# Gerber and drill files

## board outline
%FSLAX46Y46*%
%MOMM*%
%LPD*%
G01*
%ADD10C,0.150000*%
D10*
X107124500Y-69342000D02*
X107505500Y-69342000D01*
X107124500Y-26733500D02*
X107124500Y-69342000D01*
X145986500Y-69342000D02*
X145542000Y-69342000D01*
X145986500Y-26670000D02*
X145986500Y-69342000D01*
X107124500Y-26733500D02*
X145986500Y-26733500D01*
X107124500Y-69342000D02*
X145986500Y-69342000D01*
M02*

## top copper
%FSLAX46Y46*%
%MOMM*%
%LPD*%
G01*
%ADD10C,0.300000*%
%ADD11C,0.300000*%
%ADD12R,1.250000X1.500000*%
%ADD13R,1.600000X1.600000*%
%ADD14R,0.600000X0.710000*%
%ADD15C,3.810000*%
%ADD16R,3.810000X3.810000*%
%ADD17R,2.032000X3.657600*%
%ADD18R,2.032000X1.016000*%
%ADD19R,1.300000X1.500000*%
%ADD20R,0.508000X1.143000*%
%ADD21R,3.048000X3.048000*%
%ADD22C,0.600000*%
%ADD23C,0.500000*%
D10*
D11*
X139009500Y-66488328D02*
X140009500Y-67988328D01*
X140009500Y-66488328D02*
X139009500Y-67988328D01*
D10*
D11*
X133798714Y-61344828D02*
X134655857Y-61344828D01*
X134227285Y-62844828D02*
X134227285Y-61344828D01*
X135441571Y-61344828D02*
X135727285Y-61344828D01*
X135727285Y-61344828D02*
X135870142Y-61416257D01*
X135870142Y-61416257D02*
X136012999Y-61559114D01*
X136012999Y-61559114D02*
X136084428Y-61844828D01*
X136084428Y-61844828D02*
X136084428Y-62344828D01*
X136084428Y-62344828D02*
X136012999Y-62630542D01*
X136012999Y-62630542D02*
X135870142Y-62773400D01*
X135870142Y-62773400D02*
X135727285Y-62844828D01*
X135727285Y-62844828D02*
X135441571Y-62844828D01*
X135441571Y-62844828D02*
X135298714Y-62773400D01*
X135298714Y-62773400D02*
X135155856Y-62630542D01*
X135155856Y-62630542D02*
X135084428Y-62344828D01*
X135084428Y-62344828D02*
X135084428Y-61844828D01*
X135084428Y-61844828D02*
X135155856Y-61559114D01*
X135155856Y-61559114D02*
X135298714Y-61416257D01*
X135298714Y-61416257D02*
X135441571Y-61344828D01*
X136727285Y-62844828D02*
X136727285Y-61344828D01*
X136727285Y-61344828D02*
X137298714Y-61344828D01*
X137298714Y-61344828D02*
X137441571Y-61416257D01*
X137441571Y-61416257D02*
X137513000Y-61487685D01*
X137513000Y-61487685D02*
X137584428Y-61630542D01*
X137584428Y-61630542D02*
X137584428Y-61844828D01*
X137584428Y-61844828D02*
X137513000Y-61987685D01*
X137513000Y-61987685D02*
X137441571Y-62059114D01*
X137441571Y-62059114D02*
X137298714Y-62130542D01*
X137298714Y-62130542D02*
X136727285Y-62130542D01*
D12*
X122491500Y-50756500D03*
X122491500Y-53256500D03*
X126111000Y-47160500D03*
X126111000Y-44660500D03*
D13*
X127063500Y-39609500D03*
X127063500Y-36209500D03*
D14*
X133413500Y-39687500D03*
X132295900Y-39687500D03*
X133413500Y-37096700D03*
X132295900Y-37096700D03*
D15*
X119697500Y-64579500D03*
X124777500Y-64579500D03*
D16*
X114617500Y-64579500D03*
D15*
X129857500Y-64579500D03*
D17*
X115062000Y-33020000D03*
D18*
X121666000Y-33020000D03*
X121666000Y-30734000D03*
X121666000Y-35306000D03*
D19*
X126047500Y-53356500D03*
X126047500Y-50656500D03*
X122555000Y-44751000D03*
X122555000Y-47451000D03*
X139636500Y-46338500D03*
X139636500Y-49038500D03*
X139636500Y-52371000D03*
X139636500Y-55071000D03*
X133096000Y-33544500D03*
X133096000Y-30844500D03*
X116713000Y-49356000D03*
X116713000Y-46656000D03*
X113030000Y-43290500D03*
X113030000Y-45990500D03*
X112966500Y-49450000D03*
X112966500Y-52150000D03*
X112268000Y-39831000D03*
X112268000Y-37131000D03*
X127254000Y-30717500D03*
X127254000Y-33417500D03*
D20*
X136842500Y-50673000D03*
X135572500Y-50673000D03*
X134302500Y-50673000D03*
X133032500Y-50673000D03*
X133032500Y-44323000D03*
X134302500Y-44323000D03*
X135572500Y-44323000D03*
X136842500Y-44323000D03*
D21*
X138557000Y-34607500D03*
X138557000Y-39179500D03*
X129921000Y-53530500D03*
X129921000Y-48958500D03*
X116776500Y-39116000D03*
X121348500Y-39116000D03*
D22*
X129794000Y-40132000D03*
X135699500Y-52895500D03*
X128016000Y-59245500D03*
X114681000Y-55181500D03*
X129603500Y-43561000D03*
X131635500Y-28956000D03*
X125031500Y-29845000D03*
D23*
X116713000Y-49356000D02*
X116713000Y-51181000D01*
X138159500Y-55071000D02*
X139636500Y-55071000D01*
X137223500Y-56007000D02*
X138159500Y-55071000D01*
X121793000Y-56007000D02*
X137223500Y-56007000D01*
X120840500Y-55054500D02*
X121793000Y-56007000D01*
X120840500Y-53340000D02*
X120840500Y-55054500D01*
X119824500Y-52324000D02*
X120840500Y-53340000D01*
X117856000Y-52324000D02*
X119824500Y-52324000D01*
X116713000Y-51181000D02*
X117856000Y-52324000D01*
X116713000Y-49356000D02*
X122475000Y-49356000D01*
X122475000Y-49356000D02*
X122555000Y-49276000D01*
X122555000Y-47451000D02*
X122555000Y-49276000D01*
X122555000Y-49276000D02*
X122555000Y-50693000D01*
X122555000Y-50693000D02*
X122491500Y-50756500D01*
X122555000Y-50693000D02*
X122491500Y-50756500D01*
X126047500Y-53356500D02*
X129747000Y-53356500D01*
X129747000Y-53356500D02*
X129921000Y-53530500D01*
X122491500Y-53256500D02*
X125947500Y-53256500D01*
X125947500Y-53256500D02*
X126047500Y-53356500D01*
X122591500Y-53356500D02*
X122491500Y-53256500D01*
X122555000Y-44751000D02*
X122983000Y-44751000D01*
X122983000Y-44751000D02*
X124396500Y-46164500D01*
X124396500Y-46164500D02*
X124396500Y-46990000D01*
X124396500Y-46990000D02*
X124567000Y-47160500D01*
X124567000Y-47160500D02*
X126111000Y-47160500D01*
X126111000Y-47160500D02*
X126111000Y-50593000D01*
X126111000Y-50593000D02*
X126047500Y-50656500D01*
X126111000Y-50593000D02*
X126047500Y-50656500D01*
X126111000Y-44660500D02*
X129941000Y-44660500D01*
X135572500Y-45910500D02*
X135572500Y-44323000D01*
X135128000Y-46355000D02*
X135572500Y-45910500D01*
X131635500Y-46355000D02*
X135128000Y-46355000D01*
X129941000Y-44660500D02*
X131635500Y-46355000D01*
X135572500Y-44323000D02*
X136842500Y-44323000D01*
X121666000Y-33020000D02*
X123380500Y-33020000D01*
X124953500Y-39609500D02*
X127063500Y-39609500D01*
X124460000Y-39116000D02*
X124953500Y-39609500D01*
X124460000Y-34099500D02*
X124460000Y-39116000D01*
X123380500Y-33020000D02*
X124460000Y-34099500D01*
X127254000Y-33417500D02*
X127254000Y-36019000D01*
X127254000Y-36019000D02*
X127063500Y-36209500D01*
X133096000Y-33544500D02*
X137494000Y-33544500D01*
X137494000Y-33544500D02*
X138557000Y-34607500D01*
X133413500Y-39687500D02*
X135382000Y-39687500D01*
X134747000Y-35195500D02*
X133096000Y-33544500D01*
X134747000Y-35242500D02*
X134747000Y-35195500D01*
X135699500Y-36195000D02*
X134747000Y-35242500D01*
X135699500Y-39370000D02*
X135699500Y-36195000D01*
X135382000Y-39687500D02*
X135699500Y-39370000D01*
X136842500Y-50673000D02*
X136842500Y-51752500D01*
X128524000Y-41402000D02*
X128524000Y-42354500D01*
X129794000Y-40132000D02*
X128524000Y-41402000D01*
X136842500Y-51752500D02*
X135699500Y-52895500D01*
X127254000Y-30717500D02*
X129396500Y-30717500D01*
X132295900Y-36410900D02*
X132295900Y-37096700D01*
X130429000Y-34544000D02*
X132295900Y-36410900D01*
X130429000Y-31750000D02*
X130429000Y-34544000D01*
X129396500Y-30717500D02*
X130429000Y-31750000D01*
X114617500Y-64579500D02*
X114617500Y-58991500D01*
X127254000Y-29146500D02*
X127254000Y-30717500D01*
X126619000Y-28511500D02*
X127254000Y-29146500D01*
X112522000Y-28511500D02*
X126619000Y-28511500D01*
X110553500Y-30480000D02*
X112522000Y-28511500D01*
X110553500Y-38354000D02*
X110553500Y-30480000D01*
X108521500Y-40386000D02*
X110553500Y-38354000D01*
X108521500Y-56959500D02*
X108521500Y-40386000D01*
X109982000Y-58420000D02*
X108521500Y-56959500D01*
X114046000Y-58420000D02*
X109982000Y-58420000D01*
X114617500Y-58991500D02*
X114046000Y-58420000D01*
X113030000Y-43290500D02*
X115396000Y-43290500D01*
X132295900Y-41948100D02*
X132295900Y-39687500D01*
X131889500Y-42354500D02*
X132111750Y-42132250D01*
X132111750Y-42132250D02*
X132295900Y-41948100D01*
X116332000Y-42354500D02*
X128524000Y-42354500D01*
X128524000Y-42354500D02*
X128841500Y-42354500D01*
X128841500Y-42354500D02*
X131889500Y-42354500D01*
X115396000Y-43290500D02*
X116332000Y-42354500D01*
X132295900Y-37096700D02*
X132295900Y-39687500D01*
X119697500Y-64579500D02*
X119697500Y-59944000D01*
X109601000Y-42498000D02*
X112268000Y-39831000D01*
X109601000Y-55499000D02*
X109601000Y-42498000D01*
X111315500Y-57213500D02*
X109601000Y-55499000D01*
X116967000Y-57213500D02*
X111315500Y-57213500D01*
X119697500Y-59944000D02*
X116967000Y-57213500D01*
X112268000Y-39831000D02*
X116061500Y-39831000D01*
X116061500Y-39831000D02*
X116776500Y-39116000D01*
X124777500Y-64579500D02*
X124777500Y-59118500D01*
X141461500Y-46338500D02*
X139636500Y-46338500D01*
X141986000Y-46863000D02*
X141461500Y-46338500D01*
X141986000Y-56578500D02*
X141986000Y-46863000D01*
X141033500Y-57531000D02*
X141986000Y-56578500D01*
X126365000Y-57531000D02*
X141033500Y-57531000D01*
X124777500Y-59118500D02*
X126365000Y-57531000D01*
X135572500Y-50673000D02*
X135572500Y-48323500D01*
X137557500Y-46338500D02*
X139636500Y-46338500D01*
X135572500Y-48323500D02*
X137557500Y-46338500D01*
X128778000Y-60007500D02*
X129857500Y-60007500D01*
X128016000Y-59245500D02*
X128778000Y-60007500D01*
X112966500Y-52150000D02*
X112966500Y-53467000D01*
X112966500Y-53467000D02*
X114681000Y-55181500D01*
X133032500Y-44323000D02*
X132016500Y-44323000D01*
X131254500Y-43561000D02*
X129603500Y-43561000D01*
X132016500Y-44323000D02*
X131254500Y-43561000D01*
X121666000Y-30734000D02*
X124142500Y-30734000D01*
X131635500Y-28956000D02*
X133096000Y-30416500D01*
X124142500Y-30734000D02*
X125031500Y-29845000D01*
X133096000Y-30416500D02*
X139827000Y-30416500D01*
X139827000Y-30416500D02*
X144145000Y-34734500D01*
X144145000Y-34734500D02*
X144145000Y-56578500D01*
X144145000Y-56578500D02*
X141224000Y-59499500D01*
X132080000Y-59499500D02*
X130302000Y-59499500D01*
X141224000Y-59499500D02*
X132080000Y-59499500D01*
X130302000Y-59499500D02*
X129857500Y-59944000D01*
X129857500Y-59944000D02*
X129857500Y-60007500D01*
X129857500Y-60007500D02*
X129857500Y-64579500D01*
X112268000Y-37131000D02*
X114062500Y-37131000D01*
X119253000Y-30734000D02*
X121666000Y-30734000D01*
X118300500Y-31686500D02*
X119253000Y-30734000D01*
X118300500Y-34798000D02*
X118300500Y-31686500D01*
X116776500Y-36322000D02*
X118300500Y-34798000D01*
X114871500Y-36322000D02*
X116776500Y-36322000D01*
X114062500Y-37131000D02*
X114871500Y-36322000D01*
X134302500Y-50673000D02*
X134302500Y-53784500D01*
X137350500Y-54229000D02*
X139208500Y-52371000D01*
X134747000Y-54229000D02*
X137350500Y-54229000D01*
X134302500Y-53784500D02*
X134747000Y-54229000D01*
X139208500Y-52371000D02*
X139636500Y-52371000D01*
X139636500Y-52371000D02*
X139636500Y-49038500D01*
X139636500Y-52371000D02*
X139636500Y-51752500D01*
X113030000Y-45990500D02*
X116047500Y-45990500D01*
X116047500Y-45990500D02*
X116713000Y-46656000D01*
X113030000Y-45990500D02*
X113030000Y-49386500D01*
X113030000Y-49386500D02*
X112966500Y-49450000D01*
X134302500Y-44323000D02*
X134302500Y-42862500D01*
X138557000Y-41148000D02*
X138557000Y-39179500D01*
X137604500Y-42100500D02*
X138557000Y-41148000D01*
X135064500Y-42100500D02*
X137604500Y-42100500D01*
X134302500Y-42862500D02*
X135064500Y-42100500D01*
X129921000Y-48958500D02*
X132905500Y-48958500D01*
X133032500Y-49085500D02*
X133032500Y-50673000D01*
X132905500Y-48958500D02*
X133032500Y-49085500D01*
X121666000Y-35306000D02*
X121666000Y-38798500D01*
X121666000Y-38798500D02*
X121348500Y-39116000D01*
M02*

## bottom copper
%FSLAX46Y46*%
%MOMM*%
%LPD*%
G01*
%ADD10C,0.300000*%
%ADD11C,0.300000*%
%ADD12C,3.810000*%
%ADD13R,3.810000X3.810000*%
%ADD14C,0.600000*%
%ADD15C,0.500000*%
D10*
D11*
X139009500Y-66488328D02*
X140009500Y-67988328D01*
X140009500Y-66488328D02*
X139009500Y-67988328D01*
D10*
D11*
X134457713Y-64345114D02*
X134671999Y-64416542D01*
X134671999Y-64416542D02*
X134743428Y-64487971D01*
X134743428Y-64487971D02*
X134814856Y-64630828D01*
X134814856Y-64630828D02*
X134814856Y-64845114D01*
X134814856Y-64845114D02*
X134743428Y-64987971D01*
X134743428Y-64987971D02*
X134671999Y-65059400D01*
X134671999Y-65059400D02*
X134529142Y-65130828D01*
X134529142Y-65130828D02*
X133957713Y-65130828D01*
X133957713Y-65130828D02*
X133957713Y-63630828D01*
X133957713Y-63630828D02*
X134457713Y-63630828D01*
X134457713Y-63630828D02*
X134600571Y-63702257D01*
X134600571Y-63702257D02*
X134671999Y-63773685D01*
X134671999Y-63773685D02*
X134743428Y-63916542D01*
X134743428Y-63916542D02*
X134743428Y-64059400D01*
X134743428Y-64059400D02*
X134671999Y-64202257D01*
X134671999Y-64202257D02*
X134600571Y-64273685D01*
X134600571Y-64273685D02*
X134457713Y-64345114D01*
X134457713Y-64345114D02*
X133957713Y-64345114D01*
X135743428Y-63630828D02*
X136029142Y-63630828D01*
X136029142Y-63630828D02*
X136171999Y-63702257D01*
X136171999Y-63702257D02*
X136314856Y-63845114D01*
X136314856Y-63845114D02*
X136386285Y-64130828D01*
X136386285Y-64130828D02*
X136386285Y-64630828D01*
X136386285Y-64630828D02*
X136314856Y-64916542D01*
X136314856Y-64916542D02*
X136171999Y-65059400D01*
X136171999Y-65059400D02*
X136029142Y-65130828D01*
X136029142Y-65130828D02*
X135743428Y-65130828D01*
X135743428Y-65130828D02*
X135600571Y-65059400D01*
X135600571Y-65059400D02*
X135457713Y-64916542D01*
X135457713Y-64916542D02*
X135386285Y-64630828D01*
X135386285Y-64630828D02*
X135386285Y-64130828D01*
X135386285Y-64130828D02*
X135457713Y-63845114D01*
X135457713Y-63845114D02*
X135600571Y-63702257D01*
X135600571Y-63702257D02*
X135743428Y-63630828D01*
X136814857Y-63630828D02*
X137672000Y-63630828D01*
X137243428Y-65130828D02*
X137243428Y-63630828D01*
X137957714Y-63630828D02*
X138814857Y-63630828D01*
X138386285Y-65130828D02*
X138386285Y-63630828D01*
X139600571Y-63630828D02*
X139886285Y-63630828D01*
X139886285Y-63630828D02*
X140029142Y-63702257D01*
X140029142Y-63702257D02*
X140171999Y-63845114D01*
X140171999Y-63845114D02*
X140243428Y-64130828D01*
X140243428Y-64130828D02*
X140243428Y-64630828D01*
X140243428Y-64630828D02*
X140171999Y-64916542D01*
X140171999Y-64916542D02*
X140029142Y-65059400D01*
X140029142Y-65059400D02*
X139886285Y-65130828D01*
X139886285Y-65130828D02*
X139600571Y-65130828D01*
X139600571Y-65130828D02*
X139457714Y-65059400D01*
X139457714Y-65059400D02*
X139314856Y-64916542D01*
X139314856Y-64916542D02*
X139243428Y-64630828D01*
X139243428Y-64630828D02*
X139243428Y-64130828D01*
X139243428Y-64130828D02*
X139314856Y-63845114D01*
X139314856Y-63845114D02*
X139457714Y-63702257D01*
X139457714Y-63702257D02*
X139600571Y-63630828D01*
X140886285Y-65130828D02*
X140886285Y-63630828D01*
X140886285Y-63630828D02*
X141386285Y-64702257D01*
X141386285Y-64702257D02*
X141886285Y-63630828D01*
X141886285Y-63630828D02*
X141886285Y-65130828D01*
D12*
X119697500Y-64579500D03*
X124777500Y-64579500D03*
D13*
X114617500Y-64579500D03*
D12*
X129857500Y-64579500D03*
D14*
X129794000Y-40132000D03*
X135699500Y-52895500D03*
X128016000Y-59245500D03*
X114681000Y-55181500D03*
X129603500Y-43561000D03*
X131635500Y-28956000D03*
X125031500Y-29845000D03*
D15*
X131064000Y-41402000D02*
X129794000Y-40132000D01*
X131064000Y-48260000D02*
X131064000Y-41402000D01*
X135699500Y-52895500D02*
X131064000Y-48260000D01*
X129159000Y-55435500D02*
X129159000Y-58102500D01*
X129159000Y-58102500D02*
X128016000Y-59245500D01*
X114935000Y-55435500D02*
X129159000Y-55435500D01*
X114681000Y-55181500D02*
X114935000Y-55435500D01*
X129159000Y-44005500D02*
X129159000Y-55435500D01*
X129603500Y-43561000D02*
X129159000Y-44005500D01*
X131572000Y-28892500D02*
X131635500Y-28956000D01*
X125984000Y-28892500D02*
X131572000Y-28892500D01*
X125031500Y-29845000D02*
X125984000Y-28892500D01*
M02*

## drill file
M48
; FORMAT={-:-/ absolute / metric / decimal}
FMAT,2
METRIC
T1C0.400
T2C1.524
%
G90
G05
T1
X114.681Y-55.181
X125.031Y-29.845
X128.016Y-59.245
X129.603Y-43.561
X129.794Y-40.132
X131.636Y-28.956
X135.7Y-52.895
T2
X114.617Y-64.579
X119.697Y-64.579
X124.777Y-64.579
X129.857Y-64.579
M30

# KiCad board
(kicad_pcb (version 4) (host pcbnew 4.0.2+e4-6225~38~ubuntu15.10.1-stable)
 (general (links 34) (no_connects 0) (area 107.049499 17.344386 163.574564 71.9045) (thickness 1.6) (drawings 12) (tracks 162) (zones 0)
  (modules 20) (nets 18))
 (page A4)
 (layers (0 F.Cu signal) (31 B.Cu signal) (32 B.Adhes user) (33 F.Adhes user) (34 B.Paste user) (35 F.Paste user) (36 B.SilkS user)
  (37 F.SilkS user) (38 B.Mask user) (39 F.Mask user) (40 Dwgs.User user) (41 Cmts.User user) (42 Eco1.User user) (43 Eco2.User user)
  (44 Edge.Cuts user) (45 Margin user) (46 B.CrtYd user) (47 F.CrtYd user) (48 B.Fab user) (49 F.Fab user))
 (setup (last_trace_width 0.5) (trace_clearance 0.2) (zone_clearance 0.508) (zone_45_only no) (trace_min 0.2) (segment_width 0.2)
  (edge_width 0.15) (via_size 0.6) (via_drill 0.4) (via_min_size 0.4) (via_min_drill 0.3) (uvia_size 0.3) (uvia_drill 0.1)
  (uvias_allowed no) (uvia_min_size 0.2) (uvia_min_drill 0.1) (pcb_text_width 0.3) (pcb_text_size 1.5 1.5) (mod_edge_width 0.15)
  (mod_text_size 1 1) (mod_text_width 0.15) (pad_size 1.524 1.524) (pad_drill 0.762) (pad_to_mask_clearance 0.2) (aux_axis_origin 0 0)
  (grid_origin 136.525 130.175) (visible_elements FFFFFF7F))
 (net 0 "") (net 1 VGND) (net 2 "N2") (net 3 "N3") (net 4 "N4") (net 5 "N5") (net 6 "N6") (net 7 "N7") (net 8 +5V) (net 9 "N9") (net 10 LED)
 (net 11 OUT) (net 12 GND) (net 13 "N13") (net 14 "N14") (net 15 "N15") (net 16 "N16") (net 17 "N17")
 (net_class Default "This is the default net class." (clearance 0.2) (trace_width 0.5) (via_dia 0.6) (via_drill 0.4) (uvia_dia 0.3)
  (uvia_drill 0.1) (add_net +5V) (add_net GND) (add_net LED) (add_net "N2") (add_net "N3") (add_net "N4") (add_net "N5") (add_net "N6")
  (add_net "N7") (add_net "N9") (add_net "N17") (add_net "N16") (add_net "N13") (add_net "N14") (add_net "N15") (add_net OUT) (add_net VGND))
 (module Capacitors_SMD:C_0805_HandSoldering (layer F.Cu) (at 122.4915 52.0065 270)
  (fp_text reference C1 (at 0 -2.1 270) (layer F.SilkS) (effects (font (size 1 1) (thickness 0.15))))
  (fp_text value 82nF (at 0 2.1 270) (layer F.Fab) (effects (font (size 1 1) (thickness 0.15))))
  (pad 1 smd rect (at -1.25 0 270) (size 1.5 1.25) (layers F.Cu F.Paste F.Mask) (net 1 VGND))
  (pad 2 smd rect (at 1.25 0 270) (size 1.5 1.25) (layers F.Cu F.Paste F.Mask) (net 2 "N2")))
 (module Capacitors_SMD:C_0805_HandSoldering (layer F.Cu) (at 126.111 45.9105 90)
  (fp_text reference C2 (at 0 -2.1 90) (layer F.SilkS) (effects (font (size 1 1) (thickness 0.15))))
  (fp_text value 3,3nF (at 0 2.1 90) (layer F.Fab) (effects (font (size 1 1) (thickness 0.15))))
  (pad 1 smd rect (at -1.25 0 90) (size 1.5 1.25) (layers F.Cu F.Paste F.Mask) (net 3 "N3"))
  (pad 2 smd rect (at 1.25 0 90) (size 1.5 1.25) (layers F.Cu F.Paste F.Mask) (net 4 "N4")))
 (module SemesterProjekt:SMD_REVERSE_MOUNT (layer F.Cu) (at 127.0635 37.9095 90)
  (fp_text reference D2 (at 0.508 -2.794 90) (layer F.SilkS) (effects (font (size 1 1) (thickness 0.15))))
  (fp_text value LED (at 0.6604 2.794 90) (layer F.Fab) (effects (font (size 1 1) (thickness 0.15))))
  (pad 1 smd rect (at -1.7 0 90) (size 1.6 1.6) (layers F.Cu F.Paste F.Mask) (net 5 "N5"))
  (pad 2 smd rect (at 1.7 0 90) (size 1.6 1.6) (layers F.Cu F.Paste F.Mask) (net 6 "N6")))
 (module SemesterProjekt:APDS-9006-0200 (layer F.Cu) (at 133.4135 39.6875 180)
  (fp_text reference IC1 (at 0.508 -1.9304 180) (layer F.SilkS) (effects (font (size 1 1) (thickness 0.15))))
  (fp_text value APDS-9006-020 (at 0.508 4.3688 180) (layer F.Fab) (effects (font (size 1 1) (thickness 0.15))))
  (pad 1 smd rect (at 0 0 180) (size 0.6 0.71) (layers F.Cu F.Paste F.Mask) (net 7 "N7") (solder_mask_margin 0.15) (clearance 0.15))
  (pad 2 smd rect (at 1.1176 0 180) (size 0.6 0.71) (layers F.Cu F.Paste F.Mask) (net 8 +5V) (solder_mask_margin 0.15) (clearance 0.15))
  (pad 4 smd rect (at 0 2.5908 180) (size 0.6 0.71) (layers F.Cu F.Paste F.Mask) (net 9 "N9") (solder_mask_margin 0.15) (clearance 0.15))
  (pad 3 smd rect (at 1.1176 2.5908 180) (size 0.6 0.71) (layers F.Cu F.Paste F.Mask) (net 8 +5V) (solder_mask_margin 0.15) (clearance 0.15)))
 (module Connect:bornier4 (layer B.Cu) (at 122.2375 64.5795)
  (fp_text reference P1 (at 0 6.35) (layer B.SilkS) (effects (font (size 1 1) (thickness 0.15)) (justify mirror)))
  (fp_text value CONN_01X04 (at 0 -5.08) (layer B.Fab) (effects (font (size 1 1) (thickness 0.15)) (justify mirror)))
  (pad 2 thru_hole circle (at -2.54 0) (size 3.81 3.81) (drill 1.524) (layers *.Cu *.Mask B.SilkS) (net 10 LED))
  (pad 3 thru_hole circle (at 2.54 0) (size 3.81 3.81) (drill 1.524) (layers *.Cu *.Mask B.SilkS) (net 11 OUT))
  (pad 1 thru_hole rect (at -7.62 0) (size 3.81 3.81) (drill 1.524) (layers *.Cu *.Mask B.SilkS) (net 8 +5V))
  (pad 4 thru_hole circle (at 7.62 0) (size 3.81 3.81) (drill 1.524) (layers *.Cu *.Mask B.SilkS) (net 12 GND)))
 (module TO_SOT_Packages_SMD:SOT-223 (layer F.Cu) (at 118.364 33.02 90)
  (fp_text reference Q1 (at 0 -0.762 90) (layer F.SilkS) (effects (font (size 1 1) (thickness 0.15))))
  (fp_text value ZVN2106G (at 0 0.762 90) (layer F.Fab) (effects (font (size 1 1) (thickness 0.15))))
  (pad 4 smd rect (at 0 -3.302 90) (size 3.6576 2.032) (layers F.Cu F.Paste F.Mask))
  (pad 2 smd rect (at 0 3.302 90) (size 1.016 2.032) (layers F.Cu F.Paste F.Mask) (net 5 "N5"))
  (pad 3 smd rect (at 2.286 3.302 90) (size 1.016 2.032) (layers F.Cu F.Paste F.Mask) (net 12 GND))
  (pad 1 smd rect (at -2.286 3.302 90) (size 1.016 2.032) (layers F.Cu F.Paste F.Mask) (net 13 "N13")))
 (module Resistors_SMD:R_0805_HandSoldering (layer F.Cu) (at 126.0475 52.0065 90)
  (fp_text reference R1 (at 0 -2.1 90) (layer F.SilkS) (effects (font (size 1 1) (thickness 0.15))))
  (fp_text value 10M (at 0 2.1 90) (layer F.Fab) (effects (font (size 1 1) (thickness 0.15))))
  (pad 1 smd rect (at -1.35 0 90) (size 1.5 1.3) (layers F.Cu F.Paste F.Mask) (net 2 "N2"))
  (pad 2 smd rect (at 1.35 0 90) (size 1.5 1.3) (layers F.Cu F.Paste F.Mask) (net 3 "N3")))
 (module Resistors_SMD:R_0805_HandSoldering (layer F.Cu) (at 122.555 46.101 270)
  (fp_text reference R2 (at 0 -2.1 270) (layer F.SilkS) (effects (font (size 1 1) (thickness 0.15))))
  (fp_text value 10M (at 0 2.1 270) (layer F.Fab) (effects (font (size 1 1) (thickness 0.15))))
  (pad 1 smd rect (at -1.35 0 270) (size 1.5 1.3) (layers F.Cu F.Paste F.Mask) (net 3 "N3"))
  (pad 2 smd rect (at 1.35 0 270) (size 1.5 1.3) (layers F.Cu F.Paste F.Mask) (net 1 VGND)))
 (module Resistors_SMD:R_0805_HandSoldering (layer F.Cu) (at 139.6365 47.6885 270)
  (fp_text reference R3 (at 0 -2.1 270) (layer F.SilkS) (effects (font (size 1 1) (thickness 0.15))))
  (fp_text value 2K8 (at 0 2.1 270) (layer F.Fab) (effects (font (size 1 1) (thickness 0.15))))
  (pad 1 smd rect (at -1.35 0 270) (size 1.5 1.3) (layers F.Cu F.Paste F.Mask) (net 11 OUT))
  (pad 2 smd rect (at 1.35 0 270) (size 1.5 1.3) (layers F.Cu F.Paste F.Mask) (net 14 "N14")))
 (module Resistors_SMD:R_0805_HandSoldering (layer F.Cu) (at 139.6365 53.721 270)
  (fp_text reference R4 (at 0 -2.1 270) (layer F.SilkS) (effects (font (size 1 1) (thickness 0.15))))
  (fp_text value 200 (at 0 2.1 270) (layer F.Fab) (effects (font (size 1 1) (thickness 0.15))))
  (pad 1 smd rect (at -1.35 0 270) (size 1.5 1.3) (layers F.Cu F.Paste F.Mask) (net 14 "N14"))
  (pad 2 smd rect (at 1.35 0 270) (size 1.5 1.3) (layers F.Cu F.Paste F.Mask) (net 1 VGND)))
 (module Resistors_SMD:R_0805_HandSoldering (layer F.Cu) (at 133.096 32.1945 90)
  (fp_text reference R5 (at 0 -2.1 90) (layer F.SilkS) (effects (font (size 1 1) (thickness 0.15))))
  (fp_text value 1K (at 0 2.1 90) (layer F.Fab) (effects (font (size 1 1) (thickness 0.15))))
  (pad 1 smd rect (at -1.35 0 90) (size 1.5 1.3) (layers F.Cu F.Paste F.Mask) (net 7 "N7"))
  (pad 2 smd rect (at 1.35 0 90) (size 1.5 1.3) (layers F.Cu F.Paste F.Mask) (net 12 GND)))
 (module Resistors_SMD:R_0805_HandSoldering (layer F.Cu) (at 116.713 48.006 90)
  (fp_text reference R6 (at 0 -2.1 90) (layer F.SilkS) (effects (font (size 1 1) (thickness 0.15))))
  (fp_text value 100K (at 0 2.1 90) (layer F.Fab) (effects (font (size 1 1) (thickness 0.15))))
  (pad 1 smd rect (at -1.35 0 90) (size 1.5 1.3) (layers F.Cu F.Paste F.Mask) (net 1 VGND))
  (pad 2 smd rect (at 1.35 0 90) (size 1.5 1.3) (layers F.Cu F.Paste F.Mask) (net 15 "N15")))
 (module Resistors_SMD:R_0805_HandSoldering (layer F.Cu) (at 113.03 44.6405 270)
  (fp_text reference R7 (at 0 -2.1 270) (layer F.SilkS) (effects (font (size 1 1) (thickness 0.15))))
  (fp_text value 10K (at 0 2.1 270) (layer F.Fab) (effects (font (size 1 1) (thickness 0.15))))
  (pad 1 smd rect (at -1.35 0 270) (size 1.5 1.3) (layers F.Cu F.Paste F.Mask) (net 8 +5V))
  (pad 2 smd rect (at 1.35 0 270) (size 1.5 1.3) (layers F.Cu F.Paste F.Mask) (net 15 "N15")))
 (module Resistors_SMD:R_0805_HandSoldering (layer F.Cu) (at 112.9665 50.8 270)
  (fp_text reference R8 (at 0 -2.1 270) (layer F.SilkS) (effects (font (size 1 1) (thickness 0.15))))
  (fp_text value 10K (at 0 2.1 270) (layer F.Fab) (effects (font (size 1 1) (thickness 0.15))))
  (pad 1 smd rect (at -1.35 0 270) (size 1.5 1.3) (layers F.Cu F.Paste F.Mask) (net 15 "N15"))
  (pad 2 smd rect (at 1.35 0 270) (size 1.5 1.3) (layers F.Cu F.Paste F.Mask) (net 12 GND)))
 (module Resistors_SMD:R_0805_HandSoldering (layer F.Cu) (at 112.268 38.481 90)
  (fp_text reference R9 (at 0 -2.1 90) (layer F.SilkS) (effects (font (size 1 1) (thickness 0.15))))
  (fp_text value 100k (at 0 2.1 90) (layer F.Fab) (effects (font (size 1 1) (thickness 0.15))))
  (pad 1 smd rect (at -1.35 0 90) (size 1.5 1.3) (layers F.Cu F.Paste F.Mask) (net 10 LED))
  (pad 2 smd rect (at 1.35 0 90) (size 1.5 1.3) (layers F.Cu F.Paste F.Mask) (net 12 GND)))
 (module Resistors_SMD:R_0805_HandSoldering (layer F.Cu) (at 127.254 32.0675 270)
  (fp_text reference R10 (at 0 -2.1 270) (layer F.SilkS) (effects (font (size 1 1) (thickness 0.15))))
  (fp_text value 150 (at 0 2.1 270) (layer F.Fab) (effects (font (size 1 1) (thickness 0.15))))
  (pad 1 smd rect (at -1.35 0 270) (size 1.5 1.3) (layers F.Cu F.Paste F.Mask) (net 8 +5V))
  (pad 2 smd rect (at 1.35 0 270) (size 1.5 1.3) (layers F.Cu F.Paste F.Mask) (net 6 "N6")))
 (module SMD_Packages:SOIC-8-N (layer F.Cu) (at 134.9375 47.498 180)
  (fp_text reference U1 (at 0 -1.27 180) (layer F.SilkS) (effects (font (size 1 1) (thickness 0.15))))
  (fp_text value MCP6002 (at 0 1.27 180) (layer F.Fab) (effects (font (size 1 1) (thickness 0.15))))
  (pad 8 smd rect (at -1.905 -3.175 180) (size 0.508 1.143) (layers F.Cu F.Paste F.Mask) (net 8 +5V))
  (pad 7 smd rect (at -0.635 -3.175 180) (size 0.508 1.143) (layers F.Cu F.Paste F.Mask) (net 11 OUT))
  (pad 6 smd rect (at 0.635 -3.175 180) (size 0.508 1.143) (layers F.Cu F.Paste F.Mask) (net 14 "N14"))
  (pad 5 smd rect (at 1.905 -3.175 180) (size 0.508 1.143) (layers F.Cu F.Paste F.Mask) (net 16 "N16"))
  (pad 4 smd rect (at 1.905 3.175 180) (size 0.508 1.143) (layers F.Cu F.Paste F.Mask) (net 12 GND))
  (pad 3 smd rect (at 0.635 3.175 180) (size 0.508 1.143) (layers F.Cu F.Paste F.Mask) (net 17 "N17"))
  (pad 2 smd rect (at -0.635 3.175 180) (size 0.508 1.143) (layers F.Cu F.Paste F.Mask) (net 4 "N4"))
  (pad 1 smd rect (at -1.905 3.175 180) (size 0.508 1.143) (layers F.Cu F.Paste F.Mask) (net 4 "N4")))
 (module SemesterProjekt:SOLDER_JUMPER (layer F.Cu) (at 138.557 34.6075 270)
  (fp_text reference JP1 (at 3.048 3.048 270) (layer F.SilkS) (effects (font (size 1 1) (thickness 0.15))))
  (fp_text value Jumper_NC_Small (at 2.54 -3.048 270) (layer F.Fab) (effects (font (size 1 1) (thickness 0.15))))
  (pad 1 smd rect (at 0 0 270) (size 3.048 3.048) (layers F.Cu F.Paste F.Mask) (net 7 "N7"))
  (pad 2 smd rect (at 4.572 0 270) (size 3.048 3.048) (layers F.Cu F.Paste F.Mask) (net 17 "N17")))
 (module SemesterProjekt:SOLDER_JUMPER (layer F.Cu) (at 129.921 53.5305 90)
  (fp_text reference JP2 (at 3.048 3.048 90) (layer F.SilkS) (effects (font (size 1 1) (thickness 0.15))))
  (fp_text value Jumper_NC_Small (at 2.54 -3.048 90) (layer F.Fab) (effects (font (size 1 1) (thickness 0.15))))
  (pad 1 smd rect (at 0 0 90) (size 3.048 3.048) (layers F.Cu F.Paste F.Mask) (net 2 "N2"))
  (pad 2 smd rect (at 4.572 0 90) (size 3.048 3.048) (layers F.Cu F.Paste F.Mask) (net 16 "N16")))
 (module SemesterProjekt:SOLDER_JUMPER (layer F.Cu) (at 116.7765 39.116)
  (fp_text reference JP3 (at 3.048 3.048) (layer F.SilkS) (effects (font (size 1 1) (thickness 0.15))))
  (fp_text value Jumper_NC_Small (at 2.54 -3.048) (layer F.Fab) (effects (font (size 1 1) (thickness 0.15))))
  (pad 1 smd rect (at 0 0) (size 3.048 3.048) (layers F.Cu F.Paste F.Mask) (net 10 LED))
  (pad 2 smd rect (at 4.572 0) (size 3.048 3.048) (layers F.Cu F.Paste F.Mask) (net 13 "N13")))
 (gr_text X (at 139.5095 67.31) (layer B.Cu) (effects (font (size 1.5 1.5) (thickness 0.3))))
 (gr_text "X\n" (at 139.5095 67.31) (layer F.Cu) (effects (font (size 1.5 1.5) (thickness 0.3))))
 (gr_line (start 107.1245 69.342) (end 107.5055 69.342) (angle 90) (layer Edge.Cuts) (width 0.15))
 (gr_line (start 107.1245 26.7335) (end 107.1245 69.342) (angle 90) (layer Edge.Cuts) (width 0.15))
 (gr_line (start 145.9865 69.342) (end 145.542 69.342) (angle 90) (layer Edge.Cuts) (width 0.15))
 (gr_line (start 145.9865 26.67) (end 145.9865 69.342) (angle 90) (layer Edge.Cuts) (width 0.15))
 (gr_line (start 107.1245 26.7335) (end 145.9865 26.7335) (angle 90) (layer Edge.Cuts) (width 0.15))
 (gr_line (start 107.1245 69.342) (end 145.9865 69.342) (angle 90) (layer Edge.Cuts) (width 0.15))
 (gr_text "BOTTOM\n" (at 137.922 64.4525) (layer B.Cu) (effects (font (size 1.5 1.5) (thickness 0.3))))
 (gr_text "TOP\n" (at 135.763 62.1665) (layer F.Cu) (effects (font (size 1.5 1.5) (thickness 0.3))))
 (segment (start 116.713 49.356) (end 116.713 51.181) (width 0.5) (layer F.Cu) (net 1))
 (segment (start 138.1595 55.071) (end 139.6365 55.071) (width 0.5) (layer F.Cu) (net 1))
 (segment (start 137.2235 56.007) (end 138.1595 55.071) (width 0.5) (layer F.Cu) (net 1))
 (segment (start 121.793 56.007) (end 137.2235 56.007) (width 0.5) (layer F.Cu) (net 1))
 (segment (start 120.8405 55.0545) (end 121.793 56.007) (width 0.5) (layer F.Cu) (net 1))
 (segment (start 120.8405 53.34) (end 120.8405 55.0545) (width 0.5) (layer F.Cu) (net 1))
 (segment (start 119.8245 52.324) (end 120.8405 53.34) (width 0.5) (layer F.Cu) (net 1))
 (segment (start 117.856 52.324) (end 119.8245 52.324) (width 0.5) (layer F.Cu) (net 1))
 (segment (start 116.713 51.181) (end 117.856 52.324) (width 0.5) (layer F.Cu) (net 1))
 (segment (start 116.713 49.356) (end 122.475 49.356) (width 0.5) (layer F.Cu) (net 1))
 (segment (start 122.475 49.356) (end 122.555 49.276) (width 0.5) (layer F.Cu) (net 1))
 (segment (start 122.555 47.451) (end 122.555 49.276) (width 0.5) (layer F.Cu) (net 1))
 (segment (start 122.555 49.276) (end 122.555 50.693) (width 0.5) (layer F.Cu) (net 1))
 (segment (start 122.555 50.693) (end 122.4915 50.7565) (width 0.5) (layer F.Cu) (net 1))
 (segment (start 122.555 50.693) (end 122.4915 50.7565) (width 0.5) (layer F.Cu) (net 1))
 (segment (start 126.0475 53.3565) (end 129.747 53.3565) (width 0.5) (layer F.Cu) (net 2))
 (segment (start 129.747 53.3565) (end 129.921 53.5305) (width 0.5) (layer F.Cu) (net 2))
 (segment (start 122.4915 53.2565) (end 125.9475 53.2565) (width 0.5) (layer F.Cu) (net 2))
 (segment (start 125.9475 53.2565) (end 126.0475 53.3565) (width 0.5) (layer F.Cu) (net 2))
 (segment (start 122.5915 53.3565) (end 122.4915 53.2565) (width 0.5) (layer F.Cu) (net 2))
 (segment (start 122.555 44.751) (end 122.983 44.751) (width 0.5) (layer F.Cu) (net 3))
 (segment (start 122.983 44.751) (end 124.3965 46.1645) (width 0.5) (layer F.Cu) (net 3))
 (segment (start 124.3965 46.1645) (end 124.3965 46.99) (width 0.5) (layer F.Cu) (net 3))
 (segment (start 124.3965 46.99) (end 124.567 47.1605) (width 0.5) (layer F.Cu) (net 3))
 (segment (start 124.567 47.1605) (end 126.111 47.1605) (width 0.5) (layer F.Cu) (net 3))
 (segment (start 126.111 47.1605) (end 126.111 50.593) (width 0.5) (layer F.Cu) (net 3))
 (segment (start 126.111 50.593) (end 126.0475 50.6565) (width 0.5) (layer F.Cu) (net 3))
 (segment (start 126.111 50.593) (end 126.0475 50.6565) (width 0.5) (layer F.Cu) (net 3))
 (segment (start 126.111 44.6605) (end 129.941 44.6605) (width 0.5) (layer F.Cu) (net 4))
 (segment (start 135.5725 45.9105) (end 135.5725 44.323) (width 0.5) (layer F.Cu) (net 4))
 (segment (start 135.128 46.355) (end 135.5725 45.9105) (width 0.5) (layer F.Cu) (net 4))
 (segment (start 131.6355 46.355) (end 135.128 46.355) (width 0.5) (layer F.Cu) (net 4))
 (segment (start 129.941 44.6605) (end 131.6355 46.355) (width 0.5) (layer F.Cu) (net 4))
 (segment (start 135.5725 44.323) (end 136.8425 44.323) (width 0.5) (layer F.Cu) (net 4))
 (segment (start 121.666 33.02) (end 123.3805 33.02) (width 0.5) (layer F.Cu) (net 5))
 (segment (start 124.9535 39.6095) (end 127.0635 39.6095) (width 0.5) (layer F.Cu) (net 5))
 (segment (start 124.46 39.116) (end 124.9535 39.6095) (width 0.5) (layer F.Cu) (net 5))
 (segment (start 124.46 34.0995) (end 124.46 39.116) (width 0.5) (layer F.Cu) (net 5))
 (segment (start 123.3805 33.02) (end 124.46 34.0995) (width 0.5) (layer F.Cu) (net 5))
 (segment (start 127.254 33.4175) (end 127.254 36.019) (width 0.5) (layer F.Cu) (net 6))
 (segment (start 127.254 36.019) (end 127.0635 36.2095) (width 0.5) (layer F.Cu) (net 6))
 (segment (start 133.096 33.5445) (end 137.494 33.5445) (width 0.5) (layer F.Cu) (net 7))
 (segment (start 137.494 33.5445) (end 138.557 34.6075) (width 0.5) (layer F.Cu) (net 7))
 (segment (start 133.4135 39.6875) (end 135.382 39.6875) (width 0.5) (layer F.Cu) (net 7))
 (segment (start 134.747 35.1955) (end 133.096 33.5445) (width 0.5) (layer F.Cu) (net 7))
 (segment (start 134.747 35.2425) (end 134.747 35.1955) (width 0.5) (layer F.Cu) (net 7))
 (segment (start 135.6995 36.195) (end 134.747 35.2425) (width 0.5) (layer F.Cu) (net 7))
 (segment (start 135.6995 39.37) (end 135.6995 36.195) (width 0.5) (layer F.Cu) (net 7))
 (segment (start 135.382 39.6875) (end 135.6995 39.37) (width 0.5) (layer F.Cu) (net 7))
 (segment (start 136.8425 50.673) (end 136.8425 51.7525) (width 0.5) (layer F.Cu) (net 8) (status 400000))
 (segment (start 128.524 41.402) (end 128.524 42.3545) (width 0.5) (layer F.Cu) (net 8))
 (segment (start 129.794 40.132) (end 128.524 41.402) (width 0.5) (layer F.Cu) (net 8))
 (via (at 129.794 40.132) (size 0.6) (drill 0.4) (layers F.Cu B.Cu) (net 8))
 (segment (start 131.064 41.402) (end 129.794 40.132) (width 0.5) (layer B.Cu) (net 8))
 (segment (start 131.064 48.26) (end 131.064 41.402) (width 0.5) (layer B.Cu) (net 8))
 (segment (start 135.6995 52.8955) (end 131.064 48.26) (width 0.5) (layer B.Cu) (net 8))
 (via (at 135.6995 52.8955) (size 0.6) (drill 0.4) (layers F.Cu B.Cu) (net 8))
 (segment (start 136.8425 51.7525) (end 135.6995 52.8955) (width 0.5) (layer F.Cu) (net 8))
 (segment (start 127.254 30.7175) (end 129.3965 30.7175) (width 0.5) (layer F.Cu) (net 8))
 (segment (start 132.2959 36.4109) (end 132.2959 37.0967) (width 0.5) (layer F.Cu) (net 8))
 (segment (start 130.429 34.544) (end 132.2959 36.4109) (width 0.5) (layer F.Cu) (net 8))
 (segment (start 130.429 31.75) (end 130.429 34.544) (width 0.5) (layer F.Cu) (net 8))
 (segment (start 129.3965 30.7175) (end 130.429 31.75) (width 0.5) (layer F.Cu) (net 8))
 (segment (start 114.6175 64.5795) (end 114.6175 58.9915) (width 0.5) (layer F.Cu) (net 8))
 (segment (start 127.254 29.1465) (end 127.254 30.7175) (width 0.5) (layer F.Cu) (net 8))
 (segment (start 126.619 28.5115) (end 127.254 29.1465) (width 0.5) (layer F.Cu) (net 8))
 (segment (start 112.522 28.5115) (end 126.619 28.5115) (width 0.5) (layer F.Cu) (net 8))
 (segment (start 110.5535 30.48) (end 112.522 28.5115) (width 0.5) (layer F.Cu) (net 8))
 (segment (start 110.5535 38.354) (end 110.5535 30.48) (width 0.5) (layer F.Cu) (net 8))
 (segment (start 108.5215 40.386) (end 110.5535 38.354) (width 0.5) (layer F.Cu) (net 8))
 (segment (start 108.5215 56.9595) (end 108.5215 40.386) (width 0.5) (layer F.Cu) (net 8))
 (segment (start 109.982 58.42) (end 108.5215 56.9595) (width 0.5) (layer F.Cu) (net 8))
 (segment (start 114.046 58.42) (end 109.982 58.42) (width 0.5) (layer F.Cu) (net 8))
 (segment (start 114.6175 58.9915) (end 114.046 58.42) (width 0.5) (layer F.Cu) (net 8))
 (segment (start 113.03 43.2905) (end 115.396 43.2905) (width 0.5) (layer F.Cu) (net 8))
 (segment (start 132.2959 41.9481) (end 132.2959 39.6875) (width 0.5) (layer F.Cu) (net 8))
 (segment (start 131.8895 42.3545) (end 132.11175 42.13225) (width 0.5) (layer F.Cu) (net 8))
 (segment (start 132.11175 42.13225) (end 132.2959 41.9481) (width 0.5) (layer F.Cu) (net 8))
 (segment (start 116.332 42.3545) (end 128.524 42.3545) (width 0.5) (layer F.Cu) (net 8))
 (segment (start 128.524 42.3545) (end 128.8415 42.3545) (width 0.5) (layer F.Cu) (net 8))
 (segment (start 128.8415 42.3545) (end 131.8895 42.3545) (width 0.5) (layer F.Cu) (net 8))
 (segment (start 115.396 43.2905) (end 116.332 42.3545) (width 0.5) (layer F.Cu) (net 8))
 (segment (start 132.2959 37.0967) (end 132.2959 39.6875) (width 0.5) (layer F.Cu) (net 8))
 (segment (start 119.6975 64.5795) (end 119.6975 59.944) (width 0.5) (layer F.Cu) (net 10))
 (segment (start 109.601 42.498) (end 112.268 39.831) (width 0.5) (layer F.Cu) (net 10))
 (segment (start 109.601 55.499) (end 109.601 42.498) (width 0.5) (layer F.Cu) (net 10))
 (segment (start 111.3155 57.2135) (end 109.601 55.499) (width 0.5) (layer F.Cu) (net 10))
 (segment (start 116.967 57.2135) (end 111.3155 57.2135) (width 0.5) (layer F.Cu) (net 10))
 (segment (start 119.6975 59.944) (end 116.967 57.2135) (width 0.5) (layer F.Cu) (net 10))
 (segment (start 112.268 39.831) (end 116.0615 39.831) (width 0.5) (layer F.Cu) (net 10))
 (segment (start 116.0615 39.831) (end 116.7765 39.116) (width 0.5) (layer F.Cu) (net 10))
 (segment (start 124.7775 64.5795) (end 124.7775 59.1185) (width 0.5) (layer F.Cu) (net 11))
 (segment (start 141.4615 46.3385) (end 139.6365 46.3385) (width 0.5) (layer F.Cu) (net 11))
 (segment (start 141.986 46.863) (end 141.4615 46.3385) (width 0.5) (layer F.Cu) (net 11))
 (segment (start 141.986 56.5785) (end 141.986 46.863) (width 0.5) (layer F.Cu) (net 11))
 (segment (start 141.0335 57.531) (end 141.986 56.5785) (width 0.5) (layer F.Cu) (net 11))
 (segment (start 126.365 57.531) (end 141.0335 57.531) (width 0.5) (layer F.Cu) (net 11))
 (segment (start 124.7775 59.1185) (end 126.365 57.531) (width 0.5) (layer F.Cu) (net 11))
 (segment (start 135.5725 50.673) (end 135.5725 48.3235) (width 0.5) (layer F.Cu) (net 11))
 (segment (start 137.5575 46.3385) (end 139.6365 46.3385) (width 0.5) (layer F.Cu) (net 11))
 (segment (start 135.5725 48.3235) (end 137.5575 46.3385) (width 0.5) (layer F.Cu) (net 11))
 (segment (start 129.159 55.4355) (end 129.159 58.1025) (width 0.5) (layer B.Cu) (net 12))
 (segment (start 128.778 60.0075) (end 129.8575 60.0075) (width 0.5) (layer F.Cu) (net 12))
 (segment (start 128.016 59.2455) (end 128.778 60.0075) (width 0.5) (layer F.Cu) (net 12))
 (via (at 128.016 59.2455) (size 0.6) (drill 0.4) (layers F.Cu B.Cu) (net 12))
 (segment (start 129.159 58.1025) (end 128.016 59.2455) (width 0.5) (layer B.Cu) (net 12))
 (segment (start 112.9665 52.15) (end 112.9665 53.467) (width 0.5) (layer F.Cu) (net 12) (status 400000))
 (segment (start 114.935 55.4355) (end 129.159 55.4355) (width 0.5) (layer B.Cu) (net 12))
 (segment (start 114.681 55.1815) (end 114.935 55.4355) (width 0.5) (layer B.Cu) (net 12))
 (via (at 114.681 55.1815) (size 0.6) (drill 0.4) (layers F.Cu B.Cu) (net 12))
 (segment (start 112.9665 53.467) (end 114.681 55.1815) (width 0.5) (layer F.Cu) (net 12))
 (segment (start 133.0325 44.323) (end 132.0165 44.323) (width 0.5) (layer F.Cu) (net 12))
 (segment (start 129.159 44.0055) (end 129.159 55.4355) (width 0.5) (layer B.Cu) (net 12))
 (segment (start 129.6035 43.561) (end 129.159 44.0055) (width 0.5) (layer B.Cu) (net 12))
 (via (at 129.6035 43.561) (size 0.6) (drill 0.4) (layers F.Cu B.Cu) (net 12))
 (segment (start 131.2545 43.561) (end 129.6035 43.561) (width 0.5) (layer F.Cu) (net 12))
 (segment (start 132.0165 44.323) (end 131.2545 43.561) (width 0.5) (layer F.Cu) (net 12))
 (segment (start 121.666 30.734) (end 124.1425 30.734) (width 0.5) (layer F.Cu) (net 12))
 (segment (start 131.6355 28.956) (end 133.096 30.4165) (width 0.5) (layer F.Cu) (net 12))
 (via (at 131.6355 28.956) (size 0.6) (drill 0.4) (layers F.Cu B.Cu) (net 12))
 (segment (start 131.572 28.8925) (end 131.6355 28.956) (width 0.5) (layer B.Cu) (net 12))
 (segment (start 125.984 28.8925) (end 131.572 28.8925) (width 0.5) (layer B.Cu) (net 12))
 (segment (start 125.0315 29.845) (end 125.984 28.8925) (width 0.5) (layer B.Cu) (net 12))
 (via (at 125.0315 29.845) (size 0.6) (drill 0.4) (layers F.Cu B.Cu) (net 12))
 (segment (start 124.1425 30.734) (end 125.0315 29.845) (width 0.5) (layer F.Cu) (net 12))
 (segment (start 133.096 30.4165) (end 139.827 30.4165) (width 0.5) (layer F.Cu) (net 12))
 (segment (start 139.827 30.4165) (end 144.145 34.7345) (width 0.5) (layer F.Cu) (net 12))
 (segment (start 144.145 34.7345) (end 144.145 56.5785) (width 0.5) (layer F.Cu) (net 12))
 (segment (start 144.145 56.5785) (end 141.224 59.4995) (width 0.5) (layer F.Cu) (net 12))
 (segment (start 132.08 59.4995) (end 130.302 59.4995) (width 0.5) (layer F.Cu) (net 12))
 (segment (start 141.224 59.4995) (end 132.08 59.4995) (width 0.5) (layer F.Cu) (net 12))
 (segment (start 130.302 59.4995) (end 129.8575 59.944) (width 0.5) (layer F.Cu) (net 12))
 (segment (start 129.8575 59.944) (end 129.8575 60.0075) (width 0.5) (layer F.Cu) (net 12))
 (segment (start 129.8575 60.0075) (end 129.8575 64.5795) (width 0.5) (layer F.Cu) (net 12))
 (segment (start 112.268 37.131) (end 114.0625 37.131) (width 0.5) (layer F.Cu) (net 12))
 (segment (start 119.253 30.734) (end 121.666 30.734) (width 0.5) (layer F.Cu) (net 12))
 (segment (start 118.3005 31.6865) (end 119.253 30.734) (width 0.5) (layer F.Cu) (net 12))
 (segment (start 118.3005 34.798) (end 118.3005 31.6865) (width 0.5) (layer F.Cu) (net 12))
 (segment (start 116.7765 36.322) (end 118.3005 34.798) (width 0.5) (layer F.Cu) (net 12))
 (segment (start 114.8715 36.322) (end 116.7765 36.322) (width 0.5) (layer F.Cu) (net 12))
 (segment (start 114.0625 37.131) (end 114.8715 36.322) (width 0.5) (layer F.Cu) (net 12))
 (segment (start 134.3025 50.673) (end 134.3025 53.7845) (width 0.5) (layer F.Cu) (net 14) (status 400000))
 (segment (start 137.3505 54.229) (end 139.2085 52.371) (width 0.5) (layer F.Cu) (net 14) (status 800000))
 (segment (start 134.747 54.229) (end 137.3505 54.229) (width 0.5) (layer F.Cu) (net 14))
 (segment (start 134.3025 53.7845) (end 134.747 54.229) (width 0.5) (layer F.Cu) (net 14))
 (segment (start 139.2085 52.371) (end 139.6365 52.371) (width 0.5) (layer F.Cu) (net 14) (status C00000))
 (segment (start 139.6365 52.371) (end 139.6365 49.0385) (width 0.5) (layer F.Cu) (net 14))
 (segment (start 139.6365 52.371) (end 139.6365 51.7525) (width 0.5) (layer F.Cu) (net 14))
 (segment (start 113.03 45.9905) (end 116.0475 45.9905) (width 0.5) (layer F.Cu) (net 15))
 (segment (start 116.0475 45.9905) (end 116.713 46.656) (width 0.5) (layer F.Cu) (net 15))
 (segment (start 113.03 45.9905) (end 113.03 49.3865) (width 0.5) (layer F.Cu) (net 15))
 (segment (start 113.03 49.3865) (end 112.9665 49.45) (width 0.5) (layer F.Cu) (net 15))
 (segment (start 134.3025 44.323) (end 134.3025 42.8625) (width 0.5) (layer F.Cu) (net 17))
 (segment (start 138.557 41.148) (end 138.557 39.1795) (width 0.5) (layer F.Cu) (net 17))
 (segment (start 137.6045 42.1005) (end 138.557 41.148) (width 0.5) (layer F.Cu) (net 17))
 (segment (start 135.0645 42.1005) (end 137.6045 42.1005) (width 0.5) (layer F.Cu) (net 17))
 (segment (start 134.3025 42.8625) (end 135.0645 42.1005) (width 0.5) (layer F.Cu) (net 17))
 (segment (start 129.921 48.9585) (end 132.9055 48.9585) (width 0.5) (layer F.Cu) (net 16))
 (segment (start 133.0325 49.0855) (end 133.0325 50.673) (width 0.5) (layer F.Cu) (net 16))
 (segment (start 132.9055 48.9585) (end 133.0325 49.0855) (width 0.5) (layer F.Cu) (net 16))
 (segment (start 121.666 35.306) (end 121.666 38.7985) (width 0.5) (layer F.Cu) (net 13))
 (segment (start 121.666 38.7985) (end 121.3485 39.116) (width 0.5) (layer F.Cu) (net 13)))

